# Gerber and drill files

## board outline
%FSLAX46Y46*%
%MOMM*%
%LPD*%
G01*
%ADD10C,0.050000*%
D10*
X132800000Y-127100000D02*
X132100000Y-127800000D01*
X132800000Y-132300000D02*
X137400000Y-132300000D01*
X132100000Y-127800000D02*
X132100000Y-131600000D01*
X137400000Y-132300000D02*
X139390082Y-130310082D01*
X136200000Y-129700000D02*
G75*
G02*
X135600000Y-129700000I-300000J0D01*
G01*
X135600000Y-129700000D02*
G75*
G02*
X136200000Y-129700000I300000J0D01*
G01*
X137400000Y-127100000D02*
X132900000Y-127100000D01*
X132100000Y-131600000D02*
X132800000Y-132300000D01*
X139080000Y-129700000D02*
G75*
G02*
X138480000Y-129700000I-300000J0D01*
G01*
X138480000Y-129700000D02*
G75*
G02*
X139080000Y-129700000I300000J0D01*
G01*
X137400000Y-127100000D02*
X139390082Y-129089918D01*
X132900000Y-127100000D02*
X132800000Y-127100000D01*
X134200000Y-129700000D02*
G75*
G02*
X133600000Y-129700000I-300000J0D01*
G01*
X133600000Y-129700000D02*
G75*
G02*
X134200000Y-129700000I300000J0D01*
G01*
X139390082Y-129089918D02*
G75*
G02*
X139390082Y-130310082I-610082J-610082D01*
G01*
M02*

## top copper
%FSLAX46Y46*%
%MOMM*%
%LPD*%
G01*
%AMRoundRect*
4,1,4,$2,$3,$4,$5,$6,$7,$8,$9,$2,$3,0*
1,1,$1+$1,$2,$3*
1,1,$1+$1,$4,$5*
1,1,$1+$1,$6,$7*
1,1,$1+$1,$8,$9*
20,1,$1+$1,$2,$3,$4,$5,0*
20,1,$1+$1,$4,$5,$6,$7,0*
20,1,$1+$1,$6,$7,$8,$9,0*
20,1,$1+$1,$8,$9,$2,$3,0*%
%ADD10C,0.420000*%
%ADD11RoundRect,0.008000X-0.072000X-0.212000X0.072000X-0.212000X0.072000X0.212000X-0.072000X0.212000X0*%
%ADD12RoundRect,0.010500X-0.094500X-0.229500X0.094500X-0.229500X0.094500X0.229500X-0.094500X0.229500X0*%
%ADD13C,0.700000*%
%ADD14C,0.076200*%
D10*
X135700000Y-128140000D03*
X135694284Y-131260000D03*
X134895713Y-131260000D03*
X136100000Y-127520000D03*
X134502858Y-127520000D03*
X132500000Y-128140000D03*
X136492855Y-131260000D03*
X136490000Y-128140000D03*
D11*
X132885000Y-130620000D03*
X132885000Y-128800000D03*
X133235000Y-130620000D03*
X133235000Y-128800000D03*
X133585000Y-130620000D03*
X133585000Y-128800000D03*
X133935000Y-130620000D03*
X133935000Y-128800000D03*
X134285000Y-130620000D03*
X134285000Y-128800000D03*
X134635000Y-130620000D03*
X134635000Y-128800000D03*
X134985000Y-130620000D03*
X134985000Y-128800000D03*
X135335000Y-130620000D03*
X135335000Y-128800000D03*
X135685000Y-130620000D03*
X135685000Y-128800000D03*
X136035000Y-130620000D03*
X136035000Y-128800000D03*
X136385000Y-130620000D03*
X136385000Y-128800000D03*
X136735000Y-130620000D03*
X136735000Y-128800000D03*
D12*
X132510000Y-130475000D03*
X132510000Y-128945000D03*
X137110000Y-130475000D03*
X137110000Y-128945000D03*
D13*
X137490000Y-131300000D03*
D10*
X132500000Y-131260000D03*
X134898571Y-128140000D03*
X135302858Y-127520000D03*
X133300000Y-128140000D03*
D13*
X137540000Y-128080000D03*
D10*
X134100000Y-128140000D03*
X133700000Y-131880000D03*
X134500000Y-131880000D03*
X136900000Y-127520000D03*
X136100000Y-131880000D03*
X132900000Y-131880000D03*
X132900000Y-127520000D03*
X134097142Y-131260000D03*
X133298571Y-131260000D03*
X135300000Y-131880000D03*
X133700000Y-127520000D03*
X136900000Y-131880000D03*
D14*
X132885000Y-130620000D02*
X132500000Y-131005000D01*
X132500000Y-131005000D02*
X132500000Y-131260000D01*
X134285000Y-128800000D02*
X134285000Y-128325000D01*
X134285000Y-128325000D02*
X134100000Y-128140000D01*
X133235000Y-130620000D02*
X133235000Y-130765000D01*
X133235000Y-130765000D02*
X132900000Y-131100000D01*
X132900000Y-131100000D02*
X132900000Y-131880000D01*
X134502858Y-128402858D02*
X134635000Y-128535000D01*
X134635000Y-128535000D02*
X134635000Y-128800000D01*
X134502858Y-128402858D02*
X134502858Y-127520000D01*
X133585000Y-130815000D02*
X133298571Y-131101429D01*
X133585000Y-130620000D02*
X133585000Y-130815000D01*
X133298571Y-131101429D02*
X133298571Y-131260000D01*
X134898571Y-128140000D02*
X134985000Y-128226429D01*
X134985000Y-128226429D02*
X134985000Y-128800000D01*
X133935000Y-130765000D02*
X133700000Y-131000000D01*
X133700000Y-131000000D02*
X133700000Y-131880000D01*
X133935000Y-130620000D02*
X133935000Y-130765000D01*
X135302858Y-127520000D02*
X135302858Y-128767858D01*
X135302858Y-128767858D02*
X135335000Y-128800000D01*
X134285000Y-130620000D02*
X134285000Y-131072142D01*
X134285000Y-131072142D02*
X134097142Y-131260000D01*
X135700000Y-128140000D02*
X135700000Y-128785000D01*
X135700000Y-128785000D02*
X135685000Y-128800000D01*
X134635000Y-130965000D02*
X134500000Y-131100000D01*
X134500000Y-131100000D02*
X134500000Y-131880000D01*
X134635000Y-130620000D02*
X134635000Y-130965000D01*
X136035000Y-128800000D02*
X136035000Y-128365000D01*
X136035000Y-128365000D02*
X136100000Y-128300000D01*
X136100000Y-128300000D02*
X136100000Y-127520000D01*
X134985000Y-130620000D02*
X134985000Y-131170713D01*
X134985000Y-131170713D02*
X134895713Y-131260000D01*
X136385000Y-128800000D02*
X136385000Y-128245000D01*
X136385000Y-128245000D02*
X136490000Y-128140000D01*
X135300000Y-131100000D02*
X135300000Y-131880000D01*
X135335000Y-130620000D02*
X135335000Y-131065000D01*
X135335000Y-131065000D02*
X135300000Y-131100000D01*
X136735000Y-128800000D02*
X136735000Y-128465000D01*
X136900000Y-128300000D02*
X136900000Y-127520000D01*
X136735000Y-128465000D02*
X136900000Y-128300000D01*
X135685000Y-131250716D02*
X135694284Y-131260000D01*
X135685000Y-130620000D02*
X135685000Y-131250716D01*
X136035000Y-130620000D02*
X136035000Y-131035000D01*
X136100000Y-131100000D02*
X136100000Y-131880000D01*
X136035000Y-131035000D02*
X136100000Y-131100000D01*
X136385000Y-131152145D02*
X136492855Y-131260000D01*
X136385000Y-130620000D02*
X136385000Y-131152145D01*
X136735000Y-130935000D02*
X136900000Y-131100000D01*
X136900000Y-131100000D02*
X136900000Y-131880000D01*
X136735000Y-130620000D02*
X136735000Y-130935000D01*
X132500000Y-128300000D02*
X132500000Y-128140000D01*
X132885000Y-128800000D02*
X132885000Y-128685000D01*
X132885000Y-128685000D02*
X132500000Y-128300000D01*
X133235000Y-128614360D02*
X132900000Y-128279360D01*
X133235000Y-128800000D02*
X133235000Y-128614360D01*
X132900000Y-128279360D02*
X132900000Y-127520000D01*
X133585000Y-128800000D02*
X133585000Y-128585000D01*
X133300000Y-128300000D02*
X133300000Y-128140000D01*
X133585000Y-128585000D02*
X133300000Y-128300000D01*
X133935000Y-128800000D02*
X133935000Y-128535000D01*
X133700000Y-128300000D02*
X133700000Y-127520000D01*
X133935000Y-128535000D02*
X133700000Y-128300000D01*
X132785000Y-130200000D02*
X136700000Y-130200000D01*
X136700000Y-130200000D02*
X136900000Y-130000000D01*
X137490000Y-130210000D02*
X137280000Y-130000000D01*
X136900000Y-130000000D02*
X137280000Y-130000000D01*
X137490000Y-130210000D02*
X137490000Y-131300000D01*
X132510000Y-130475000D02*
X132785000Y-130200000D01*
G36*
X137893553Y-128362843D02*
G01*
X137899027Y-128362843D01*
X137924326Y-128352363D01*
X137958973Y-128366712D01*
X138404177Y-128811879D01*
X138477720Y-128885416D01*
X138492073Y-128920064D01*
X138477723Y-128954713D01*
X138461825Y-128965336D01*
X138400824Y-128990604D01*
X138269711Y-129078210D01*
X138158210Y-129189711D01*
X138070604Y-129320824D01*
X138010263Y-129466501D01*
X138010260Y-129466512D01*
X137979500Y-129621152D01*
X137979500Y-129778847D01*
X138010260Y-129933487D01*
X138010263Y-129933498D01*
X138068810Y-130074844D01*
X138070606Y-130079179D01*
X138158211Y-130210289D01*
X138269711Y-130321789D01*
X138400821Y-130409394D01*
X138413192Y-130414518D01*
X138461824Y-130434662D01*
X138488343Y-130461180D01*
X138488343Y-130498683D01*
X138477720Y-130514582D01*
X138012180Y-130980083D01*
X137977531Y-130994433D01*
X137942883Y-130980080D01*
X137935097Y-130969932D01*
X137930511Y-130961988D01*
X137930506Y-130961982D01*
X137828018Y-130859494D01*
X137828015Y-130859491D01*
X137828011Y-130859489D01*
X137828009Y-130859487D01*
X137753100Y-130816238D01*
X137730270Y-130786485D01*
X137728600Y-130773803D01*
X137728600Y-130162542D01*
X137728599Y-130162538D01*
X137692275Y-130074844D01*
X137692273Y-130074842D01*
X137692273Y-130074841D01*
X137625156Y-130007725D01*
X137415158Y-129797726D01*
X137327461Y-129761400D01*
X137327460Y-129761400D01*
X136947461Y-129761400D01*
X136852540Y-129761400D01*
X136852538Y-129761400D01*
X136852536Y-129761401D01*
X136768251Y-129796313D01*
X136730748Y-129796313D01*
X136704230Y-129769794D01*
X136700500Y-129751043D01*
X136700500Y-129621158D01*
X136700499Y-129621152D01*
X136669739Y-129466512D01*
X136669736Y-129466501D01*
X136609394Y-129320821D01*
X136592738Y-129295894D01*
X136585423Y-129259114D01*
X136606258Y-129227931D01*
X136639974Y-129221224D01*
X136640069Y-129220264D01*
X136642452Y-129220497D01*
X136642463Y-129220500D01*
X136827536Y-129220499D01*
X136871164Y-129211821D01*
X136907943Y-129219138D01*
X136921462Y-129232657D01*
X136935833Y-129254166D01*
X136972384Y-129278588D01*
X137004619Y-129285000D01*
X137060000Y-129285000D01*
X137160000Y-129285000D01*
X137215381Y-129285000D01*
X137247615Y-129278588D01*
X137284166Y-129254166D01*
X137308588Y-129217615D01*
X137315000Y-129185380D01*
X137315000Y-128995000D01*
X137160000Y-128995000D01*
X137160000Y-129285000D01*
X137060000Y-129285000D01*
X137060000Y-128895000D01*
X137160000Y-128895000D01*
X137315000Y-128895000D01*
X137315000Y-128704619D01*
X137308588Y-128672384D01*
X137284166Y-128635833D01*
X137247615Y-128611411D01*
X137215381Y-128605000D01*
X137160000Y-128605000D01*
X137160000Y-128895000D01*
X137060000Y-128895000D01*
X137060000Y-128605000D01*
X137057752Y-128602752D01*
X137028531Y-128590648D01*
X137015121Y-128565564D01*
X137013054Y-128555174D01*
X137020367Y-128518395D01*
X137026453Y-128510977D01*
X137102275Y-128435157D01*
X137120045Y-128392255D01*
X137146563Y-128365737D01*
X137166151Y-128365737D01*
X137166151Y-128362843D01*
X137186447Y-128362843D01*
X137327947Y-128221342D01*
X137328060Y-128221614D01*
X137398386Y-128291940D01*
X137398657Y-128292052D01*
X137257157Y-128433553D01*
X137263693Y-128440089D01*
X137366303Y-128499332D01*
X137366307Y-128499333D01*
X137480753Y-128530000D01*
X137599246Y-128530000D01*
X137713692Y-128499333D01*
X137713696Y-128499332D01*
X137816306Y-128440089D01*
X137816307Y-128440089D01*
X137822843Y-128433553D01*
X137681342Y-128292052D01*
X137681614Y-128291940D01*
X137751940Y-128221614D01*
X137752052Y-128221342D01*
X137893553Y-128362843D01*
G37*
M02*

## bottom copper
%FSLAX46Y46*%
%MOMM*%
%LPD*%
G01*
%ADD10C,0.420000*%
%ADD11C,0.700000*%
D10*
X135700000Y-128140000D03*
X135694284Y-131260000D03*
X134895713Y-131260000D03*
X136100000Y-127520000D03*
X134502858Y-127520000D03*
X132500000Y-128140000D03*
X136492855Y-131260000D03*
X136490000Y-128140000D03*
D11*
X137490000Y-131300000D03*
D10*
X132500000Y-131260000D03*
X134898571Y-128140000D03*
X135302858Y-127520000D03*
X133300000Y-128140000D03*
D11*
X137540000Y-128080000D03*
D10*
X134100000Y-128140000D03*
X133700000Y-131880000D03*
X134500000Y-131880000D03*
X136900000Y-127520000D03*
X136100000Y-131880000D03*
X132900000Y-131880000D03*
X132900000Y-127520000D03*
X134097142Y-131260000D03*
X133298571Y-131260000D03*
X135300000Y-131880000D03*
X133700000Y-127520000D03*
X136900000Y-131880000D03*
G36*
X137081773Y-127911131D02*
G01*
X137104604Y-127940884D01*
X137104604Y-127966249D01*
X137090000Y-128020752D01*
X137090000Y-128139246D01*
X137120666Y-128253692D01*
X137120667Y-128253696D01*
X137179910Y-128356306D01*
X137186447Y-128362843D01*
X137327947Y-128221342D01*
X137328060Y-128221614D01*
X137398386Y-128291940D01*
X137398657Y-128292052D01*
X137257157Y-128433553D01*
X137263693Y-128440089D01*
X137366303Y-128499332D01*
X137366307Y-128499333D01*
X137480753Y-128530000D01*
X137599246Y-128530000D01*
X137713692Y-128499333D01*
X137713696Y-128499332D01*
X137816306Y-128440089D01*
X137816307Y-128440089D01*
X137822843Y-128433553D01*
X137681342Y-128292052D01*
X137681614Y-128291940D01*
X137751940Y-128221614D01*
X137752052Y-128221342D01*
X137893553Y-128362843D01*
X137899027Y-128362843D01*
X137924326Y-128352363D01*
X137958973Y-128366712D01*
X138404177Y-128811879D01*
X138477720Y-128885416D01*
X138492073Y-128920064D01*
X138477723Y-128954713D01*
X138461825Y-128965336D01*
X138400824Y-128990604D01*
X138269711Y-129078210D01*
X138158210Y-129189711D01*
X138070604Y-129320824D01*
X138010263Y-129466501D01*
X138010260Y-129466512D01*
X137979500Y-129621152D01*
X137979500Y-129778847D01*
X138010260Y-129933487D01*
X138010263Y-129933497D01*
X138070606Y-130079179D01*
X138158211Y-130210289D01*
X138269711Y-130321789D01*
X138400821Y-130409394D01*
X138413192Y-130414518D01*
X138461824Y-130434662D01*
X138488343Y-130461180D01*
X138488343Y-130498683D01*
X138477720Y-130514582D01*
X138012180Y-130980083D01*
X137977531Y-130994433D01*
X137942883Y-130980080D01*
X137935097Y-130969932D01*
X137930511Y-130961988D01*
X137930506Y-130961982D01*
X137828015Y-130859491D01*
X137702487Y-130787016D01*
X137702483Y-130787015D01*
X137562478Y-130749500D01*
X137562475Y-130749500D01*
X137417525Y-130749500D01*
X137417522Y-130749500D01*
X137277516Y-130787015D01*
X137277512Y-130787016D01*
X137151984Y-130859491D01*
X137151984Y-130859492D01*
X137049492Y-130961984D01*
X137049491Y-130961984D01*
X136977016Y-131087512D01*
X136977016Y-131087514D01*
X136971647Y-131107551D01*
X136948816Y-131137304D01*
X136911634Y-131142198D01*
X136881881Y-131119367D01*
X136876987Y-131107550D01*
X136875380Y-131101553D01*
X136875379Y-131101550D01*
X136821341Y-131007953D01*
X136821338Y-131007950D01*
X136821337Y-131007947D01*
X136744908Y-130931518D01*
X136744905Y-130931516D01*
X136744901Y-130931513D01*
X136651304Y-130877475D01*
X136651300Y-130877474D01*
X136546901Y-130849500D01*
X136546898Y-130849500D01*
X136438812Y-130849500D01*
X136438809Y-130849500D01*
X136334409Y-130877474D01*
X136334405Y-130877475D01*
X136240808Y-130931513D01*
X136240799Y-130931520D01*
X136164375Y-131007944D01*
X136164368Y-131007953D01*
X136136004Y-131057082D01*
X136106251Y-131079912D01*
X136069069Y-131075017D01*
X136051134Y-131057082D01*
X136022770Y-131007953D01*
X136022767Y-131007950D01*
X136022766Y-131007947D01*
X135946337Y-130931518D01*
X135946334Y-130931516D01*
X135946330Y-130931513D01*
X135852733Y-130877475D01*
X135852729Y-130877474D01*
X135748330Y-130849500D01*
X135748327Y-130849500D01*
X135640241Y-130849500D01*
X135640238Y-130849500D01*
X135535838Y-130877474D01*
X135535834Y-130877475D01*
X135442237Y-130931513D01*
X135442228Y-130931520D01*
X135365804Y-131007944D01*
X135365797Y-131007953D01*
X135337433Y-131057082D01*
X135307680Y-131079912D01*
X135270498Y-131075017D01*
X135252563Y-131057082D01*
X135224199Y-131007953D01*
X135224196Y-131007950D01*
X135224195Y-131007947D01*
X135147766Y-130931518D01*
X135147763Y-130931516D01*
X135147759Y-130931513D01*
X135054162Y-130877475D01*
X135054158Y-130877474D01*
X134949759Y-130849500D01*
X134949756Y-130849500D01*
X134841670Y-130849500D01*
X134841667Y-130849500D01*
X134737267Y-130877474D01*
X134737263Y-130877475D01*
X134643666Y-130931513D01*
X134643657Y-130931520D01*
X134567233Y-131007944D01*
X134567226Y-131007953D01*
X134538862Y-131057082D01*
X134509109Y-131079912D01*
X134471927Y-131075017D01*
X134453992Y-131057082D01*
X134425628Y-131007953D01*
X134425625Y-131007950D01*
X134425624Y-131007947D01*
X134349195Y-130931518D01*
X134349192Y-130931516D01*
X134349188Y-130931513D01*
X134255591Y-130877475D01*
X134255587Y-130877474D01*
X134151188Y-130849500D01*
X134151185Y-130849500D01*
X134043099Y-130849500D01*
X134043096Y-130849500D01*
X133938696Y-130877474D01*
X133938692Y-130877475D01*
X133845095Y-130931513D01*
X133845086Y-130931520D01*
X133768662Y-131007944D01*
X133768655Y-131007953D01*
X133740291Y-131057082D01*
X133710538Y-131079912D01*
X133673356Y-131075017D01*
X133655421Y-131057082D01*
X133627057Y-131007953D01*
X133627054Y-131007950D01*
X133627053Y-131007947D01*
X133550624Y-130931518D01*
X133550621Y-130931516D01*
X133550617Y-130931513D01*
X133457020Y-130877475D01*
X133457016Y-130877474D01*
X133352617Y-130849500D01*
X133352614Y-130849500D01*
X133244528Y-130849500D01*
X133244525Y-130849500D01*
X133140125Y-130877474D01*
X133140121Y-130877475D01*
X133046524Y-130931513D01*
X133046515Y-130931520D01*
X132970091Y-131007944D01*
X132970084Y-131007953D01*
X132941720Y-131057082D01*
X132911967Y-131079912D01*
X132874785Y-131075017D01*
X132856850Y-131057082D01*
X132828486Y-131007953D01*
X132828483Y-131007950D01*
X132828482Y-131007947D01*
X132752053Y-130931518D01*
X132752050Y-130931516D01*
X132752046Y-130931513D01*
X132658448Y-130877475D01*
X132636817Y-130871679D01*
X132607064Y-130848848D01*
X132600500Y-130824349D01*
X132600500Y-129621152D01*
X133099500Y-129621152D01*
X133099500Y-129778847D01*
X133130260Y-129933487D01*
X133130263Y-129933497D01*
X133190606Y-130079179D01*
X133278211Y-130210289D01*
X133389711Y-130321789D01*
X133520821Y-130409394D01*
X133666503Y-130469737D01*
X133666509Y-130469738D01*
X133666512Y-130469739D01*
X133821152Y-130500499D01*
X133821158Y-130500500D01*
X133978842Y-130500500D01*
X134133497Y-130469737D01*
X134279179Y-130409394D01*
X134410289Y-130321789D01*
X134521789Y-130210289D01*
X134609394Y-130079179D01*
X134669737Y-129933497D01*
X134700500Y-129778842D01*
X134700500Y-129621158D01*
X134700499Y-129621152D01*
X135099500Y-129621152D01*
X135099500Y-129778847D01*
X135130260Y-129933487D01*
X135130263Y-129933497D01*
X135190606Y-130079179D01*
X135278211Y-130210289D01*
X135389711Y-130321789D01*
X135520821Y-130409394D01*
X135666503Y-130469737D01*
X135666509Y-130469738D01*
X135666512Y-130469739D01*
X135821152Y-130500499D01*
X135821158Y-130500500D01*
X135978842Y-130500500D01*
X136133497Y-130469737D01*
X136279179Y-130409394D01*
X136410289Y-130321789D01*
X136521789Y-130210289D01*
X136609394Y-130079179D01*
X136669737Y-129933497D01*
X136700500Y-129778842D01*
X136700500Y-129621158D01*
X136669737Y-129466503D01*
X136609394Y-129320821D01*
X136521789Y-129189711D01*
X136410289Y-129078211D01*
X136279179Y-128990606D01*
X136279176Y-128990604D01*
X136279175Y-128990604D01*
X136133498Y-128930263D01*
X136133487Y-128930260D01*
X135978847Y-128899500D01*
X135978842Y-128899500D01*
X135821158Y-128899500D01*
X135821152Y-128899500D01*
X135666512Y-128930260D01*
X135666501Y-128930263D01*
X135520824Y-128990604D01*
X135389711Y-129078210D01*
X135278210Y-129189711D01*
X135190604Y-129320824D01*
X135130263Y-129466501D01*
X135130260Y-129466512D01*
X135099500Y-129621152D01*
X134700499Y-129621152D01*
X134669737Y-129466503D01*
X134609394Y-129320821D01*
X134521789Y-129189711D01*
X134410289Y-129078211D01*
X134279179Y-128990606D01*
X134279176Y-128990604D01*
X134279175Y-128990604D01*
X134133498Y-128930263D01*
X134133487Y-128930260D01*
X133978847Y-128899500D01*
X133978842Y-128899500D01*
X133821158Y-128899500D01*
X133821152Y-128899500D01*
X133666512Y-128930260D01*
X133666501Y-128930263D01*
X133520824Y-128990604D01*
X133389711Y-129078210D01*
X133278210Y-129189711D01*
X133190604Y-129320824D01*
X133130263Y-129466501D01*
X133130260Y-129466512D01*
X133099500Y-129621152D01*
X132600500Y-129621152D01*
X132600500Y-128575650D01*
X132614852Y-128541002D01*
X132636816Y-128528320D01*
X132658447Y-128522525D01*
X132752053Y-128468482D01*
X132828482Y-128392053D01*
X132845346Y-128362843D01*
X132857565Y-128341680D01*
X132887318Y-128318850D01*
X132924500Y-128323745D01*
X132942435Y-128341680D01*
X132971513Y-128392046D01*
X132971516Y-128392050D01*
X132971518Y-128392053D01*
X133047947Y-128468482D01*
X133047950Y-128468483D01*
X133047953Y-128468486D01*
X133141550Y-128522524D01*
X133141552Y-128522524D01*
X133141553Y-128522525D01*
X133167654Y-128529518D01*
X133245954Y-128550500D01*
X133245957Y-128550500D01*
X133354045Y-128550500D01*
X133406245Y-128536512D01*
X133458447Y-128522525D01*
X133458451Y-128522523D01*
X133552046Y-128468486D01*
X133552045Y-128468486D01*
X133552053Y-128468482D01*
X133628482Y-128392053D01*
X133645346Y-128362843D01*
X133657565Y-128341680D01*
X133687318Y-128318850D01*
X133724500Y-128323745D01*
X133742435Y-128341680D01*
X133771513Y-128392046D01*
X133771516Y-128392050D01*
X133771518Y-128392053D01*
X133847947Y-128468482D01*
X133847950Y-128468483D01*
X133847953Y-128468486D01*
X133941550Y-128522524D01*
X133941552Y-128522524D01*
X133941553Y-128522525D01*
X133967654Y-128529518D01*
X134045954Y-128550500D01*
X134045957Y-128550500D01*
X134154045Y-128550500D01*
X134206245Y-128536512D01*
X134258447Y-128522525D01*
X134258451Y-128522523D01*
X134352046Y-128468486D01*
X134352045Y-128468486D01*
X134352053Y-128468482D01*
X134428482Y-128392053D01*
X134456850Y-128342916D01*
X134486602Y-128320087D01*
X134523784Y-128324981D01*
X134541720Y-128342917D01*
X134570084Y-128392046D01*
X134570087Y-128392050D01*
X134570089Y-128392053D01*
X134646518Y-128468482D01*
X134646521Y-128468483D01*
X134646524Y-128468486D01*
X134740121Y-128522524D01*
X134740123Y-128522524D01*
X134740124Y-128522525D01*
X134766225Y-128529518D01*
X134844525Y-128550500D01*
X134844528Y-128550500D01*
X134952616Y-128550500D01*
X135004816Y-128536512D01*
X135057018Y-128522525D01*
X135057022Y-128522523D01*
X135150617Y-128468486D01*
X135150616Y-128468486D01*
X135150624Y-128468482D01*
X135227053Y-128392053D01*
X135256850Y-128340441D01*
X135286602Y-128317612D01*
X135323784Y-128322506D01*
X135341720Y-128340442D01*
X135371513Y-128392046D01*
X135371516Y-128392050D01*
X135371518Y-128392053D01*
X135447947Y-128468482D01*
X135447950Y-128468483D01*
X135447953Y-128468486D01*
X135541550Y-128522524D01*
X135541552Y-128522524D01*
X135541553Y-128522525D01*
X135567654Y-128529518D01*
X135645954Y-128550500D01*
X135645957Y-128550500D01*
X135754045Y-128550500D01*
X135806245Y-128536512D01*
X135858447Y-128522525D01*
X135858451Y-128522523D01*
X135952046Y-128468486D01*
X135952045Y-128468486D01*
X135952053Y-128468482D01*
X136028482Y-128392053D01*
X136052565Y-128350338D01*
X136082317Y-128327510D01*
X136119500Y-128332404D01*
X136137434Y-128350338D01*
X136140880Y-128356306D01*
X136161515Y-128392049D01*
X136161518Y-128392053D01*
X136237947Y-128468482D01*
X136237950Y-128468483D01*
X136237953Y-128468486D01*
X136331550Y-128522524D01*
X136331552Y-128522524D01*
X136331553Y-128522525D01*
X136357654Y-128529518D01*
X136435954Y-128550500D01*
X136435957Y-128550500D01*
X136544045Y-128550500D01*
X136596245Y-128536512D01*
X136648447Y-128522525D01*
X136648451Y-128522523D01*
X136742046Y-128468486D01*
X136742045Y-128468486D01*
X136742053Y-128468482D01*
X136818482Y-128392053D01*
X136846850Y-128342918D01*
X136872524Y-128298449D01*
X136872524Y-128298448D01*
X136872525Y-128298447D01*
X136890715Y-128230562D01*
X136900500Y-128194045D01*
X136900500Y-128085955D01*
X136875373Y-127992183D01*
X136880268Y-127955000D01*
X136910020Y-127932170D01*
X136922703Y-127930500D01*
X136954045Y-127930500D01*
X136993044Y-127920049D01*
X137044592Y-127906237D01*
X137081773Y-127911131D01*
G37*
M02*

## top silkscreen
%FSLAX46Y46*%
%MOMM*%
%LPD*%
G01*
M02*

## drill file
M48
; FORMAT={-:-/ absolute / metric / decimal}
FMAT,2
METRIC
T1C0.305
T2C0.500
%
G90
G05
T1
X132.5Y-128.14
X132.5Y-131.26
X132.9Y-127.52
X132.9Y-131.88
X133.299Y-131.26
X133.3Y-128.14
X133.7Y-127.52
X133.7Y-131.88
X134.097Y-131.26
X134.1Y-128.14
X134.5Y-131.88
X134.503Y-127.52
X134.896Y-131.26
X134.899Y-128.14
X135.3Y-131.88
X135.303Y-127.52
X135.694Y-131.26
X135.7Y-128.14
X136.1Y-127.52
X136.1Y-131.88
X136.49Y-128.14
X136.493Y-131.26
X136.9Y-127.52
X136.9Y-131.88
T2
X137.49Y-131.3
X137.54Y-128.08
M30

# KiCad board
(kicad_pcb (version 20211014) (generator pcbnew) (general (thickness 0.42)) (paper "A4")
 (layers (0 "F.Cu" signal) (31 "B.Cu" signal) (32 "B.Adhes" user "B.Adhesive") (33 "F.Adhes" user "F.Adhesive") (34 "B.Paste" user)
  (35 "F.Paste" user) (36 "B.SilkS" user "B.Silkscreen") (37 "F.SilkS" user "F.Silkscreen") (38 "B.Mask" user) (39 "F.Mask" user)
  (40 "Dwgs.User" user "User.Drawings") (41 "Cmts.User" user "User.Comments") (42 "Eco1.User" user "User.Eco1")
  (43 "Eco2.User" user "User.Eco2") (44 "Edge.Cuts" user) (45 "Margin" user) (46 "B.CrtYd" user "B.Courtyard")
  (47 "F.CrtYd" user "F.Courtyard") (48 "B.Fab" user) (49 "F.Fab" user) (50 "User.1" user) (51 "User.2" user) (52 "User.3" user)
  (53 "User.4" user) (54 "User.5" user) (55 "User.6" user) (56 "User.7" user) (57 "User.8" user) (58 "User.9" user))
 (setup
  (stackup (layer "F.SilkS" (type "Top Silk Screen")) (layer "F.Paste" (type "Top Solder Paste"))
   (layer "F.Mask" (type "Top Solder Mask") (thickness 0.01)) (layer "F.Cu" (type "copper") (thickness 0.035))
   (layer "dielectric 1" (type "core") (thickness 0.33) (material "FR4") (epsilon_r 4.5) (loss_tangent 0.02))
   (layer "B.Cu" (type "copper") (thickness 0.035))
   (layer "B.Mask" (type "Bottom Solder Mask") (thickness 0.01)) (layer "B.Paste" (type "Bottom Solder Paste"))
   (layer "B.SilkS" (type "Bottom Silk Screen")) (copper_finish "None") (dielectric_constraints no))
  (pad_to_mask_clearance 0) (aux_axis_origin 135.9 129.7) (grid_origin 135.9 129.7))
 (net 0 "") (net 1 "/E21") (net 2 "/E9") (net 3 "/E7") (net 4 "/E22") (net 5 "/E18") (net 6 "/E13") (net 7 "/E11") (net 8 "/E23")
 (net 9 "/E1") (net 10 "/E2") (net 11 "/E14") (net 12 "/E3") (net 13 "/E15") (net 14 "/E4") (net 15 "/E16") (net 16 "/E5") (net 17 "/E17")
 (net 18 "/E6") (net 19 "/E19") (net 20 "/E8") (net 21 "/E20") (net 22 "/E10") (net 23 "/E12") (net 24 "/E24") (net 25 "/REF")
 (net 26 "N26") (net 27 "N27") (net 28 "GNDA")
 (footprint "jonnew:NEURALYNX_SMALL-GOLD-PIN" (layer "F.Cu") (at 135.7 128.14)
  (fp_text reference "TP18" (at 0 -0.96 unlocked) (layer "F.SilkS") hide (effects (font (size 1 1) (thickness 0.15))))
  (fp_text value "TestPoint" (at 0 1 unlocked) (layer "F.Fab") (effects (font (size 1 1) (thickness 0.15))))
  (pad "1" thru_hole circle (at 0 0) (size 0.42 0.42) (drill 0.3048) (layers *.Cu *.Mask) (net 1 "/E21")))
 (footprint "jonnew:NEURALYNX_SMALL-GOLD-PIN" (layer "F.Cu") (at 135.694284 131.26)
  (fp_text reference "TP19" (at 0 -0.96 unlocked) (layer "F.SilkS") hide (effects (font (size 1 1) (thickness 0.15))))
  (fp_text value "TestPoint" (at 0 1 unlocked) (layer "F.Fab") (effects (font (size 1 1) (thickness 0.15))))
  (pad "1" thru_hole circle (at 0 0) (size 0.42 0.42) (drill 0.3048) (layers *.Cu *.Mask) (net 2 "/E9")))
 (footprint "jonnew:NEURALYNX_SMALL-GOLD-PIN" (layer "F.Cu") (at 134.895713 131.26)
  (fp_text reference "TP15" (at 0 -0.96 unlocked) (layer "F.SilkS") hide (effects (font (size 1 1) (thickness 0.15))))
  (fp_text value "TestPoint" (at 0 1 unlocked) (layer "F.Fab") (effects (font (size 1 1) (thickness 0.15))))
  (pad "1" thru_hole circle (at 0 0) (size 0.42 0.42) (drill 0.3048) (layers *.Cu *.Mask) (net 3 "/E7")))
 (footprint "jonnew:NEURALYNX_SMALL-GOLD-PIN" (layer "F.Cu") (at 136.1 127.52)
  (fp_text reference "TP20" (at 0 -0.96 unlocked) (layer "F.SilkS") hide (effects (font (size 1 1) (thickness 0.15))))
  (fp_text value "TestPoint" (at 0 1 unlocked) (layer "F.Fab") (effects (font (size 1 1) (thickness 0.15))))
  (pad "1" thru_hole circle (at 0 0) (size 0.42 0.42) (drill 0.3048) (layers *.Cu *.Mask) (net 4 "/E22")))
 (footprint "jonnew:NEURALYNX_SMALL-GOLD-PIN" (layer "F.Cu") (at 134.502858 127.52)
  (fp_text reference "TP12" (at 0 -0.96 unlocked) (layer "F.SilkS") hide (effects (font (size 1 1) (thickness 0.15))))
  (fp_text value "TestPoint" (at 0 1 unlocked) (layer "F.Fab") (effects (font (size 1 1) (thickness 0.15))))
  (pad "1" thru_hole circle (at 0 0) (size 0.42 0.42) (drill 0.3048) (layers *.Cu *.Mask) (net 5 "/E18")))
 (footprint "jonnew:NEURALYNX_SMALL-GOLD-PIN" (layer "F.Cu") (at 132.5 128.14)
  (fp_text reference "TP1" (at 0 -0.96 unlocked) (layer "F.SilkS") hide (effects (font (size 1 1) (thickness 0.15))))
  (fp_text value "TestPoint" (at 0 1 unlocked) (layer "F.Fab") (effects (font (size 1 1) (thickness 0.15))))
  (pad "1" thru_hole circle (at 0 0) (size 0.42 0.42) (drill 0.3048) (layers *.Cu *.Mask) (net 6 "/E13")))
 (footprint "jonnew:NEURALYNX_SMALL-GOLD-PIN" (layer "F.Cu") (at 136.492855 131.26)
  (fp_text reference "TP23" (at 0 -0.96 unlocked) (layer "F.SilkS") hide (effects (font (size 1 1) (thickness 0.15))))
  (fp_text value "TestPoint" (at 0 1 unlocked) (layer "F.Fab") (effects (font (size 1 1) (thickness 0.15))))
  (pad "1" thru_hole circle (at 0 0) (size 0.42 0.42) (drill 0.3048) (layers *.Cu *.Mask) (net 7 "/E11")))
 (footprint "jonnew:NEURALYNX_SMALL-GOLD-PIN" (layer "F.Cu") (at 136.49 128.14)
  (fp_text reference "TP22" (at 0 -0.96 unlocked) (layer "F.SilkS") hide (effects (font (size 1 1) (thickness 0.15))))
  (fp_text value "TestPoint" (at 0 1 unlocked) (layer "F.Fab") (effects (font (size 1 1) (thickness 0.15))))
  (pad "1" thru_hole circle (at 0 0) (size 0.42 0.42) (drill 0.3048) (layers *.Cu *.Mask) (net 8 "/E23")))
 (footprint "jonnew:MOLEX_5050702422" (layer "F.Cu") (at 134.81 129.71)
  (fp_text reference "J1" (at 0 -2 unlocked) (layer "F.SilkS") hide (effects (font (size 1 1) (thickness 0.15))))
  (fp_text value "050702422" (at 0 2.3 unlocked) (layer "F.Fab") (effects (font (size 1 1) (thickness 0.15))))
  (pad "1" smd roundrect (at -1.925 0.91) (size 0.16 0.44) (layers "F.Cu" "F.Paste" "F.Mask") (roundrect_rratio 0.05) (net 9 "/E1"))
  (pad "2" smd roundrect (at -1.925 -0.91) (size 0.16 0.44) (layers "F.Cu" "F.Paste" "F.Mask") (roundrect_rratio 0.05) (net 6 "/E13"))
  (pad "3" smd roundrect (at -1.575 0.91) (size 0.16 0.44) (layers "F.Cu" "F.Paste" "F.Mask") (roundrect_rratio 0.05) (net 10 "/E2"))
  (pad "4" smd roundrect (at -1.575 -0.91) (size 0.16 0.44) (layers "F.Cu" "F.Paste" "F.Mask") (roundrect_rratio 0.05) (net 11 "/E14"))
  (pad "5" smd roundrect (at -1.225 0.91) (size 0.16 0.44) (layers "F.Cu" "F.Paste" "F.Mask") (roundrect_rratio 0.05) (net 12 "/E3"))
  (pad "6" smd roundrect (at -1.225 -0.91) (size 0.16 0.44) (layers "F.Cu" "F.Paste" "F.Mask") (roundrect_rratio 0.05) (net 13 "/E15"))
  (pad "7" smd roundrect (at -0.875 0.91) (size 0.16 0.44) (layers "F.Cu" "F.Paste" "F.Mask") (roundrect_rratio 0.05) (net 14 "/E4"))
  (pad "8" smd roundrect (at -0.875 -0.91) (size 0.16 0.44) (layers "F.Cu" "F.Paste" "F.Mask") (roundrect_rratio 0.05) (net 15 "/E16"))
  (pad "9" smd roundrect (at -0.525 0.91) (size 0.16 0.44) (layers "F.Cu" "F.Paste" "F.Mask") (roundrect_rratio 0.05) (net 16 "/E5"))
  (pad "10" smd roundrect (at -0.525 -0.91) (size 0.16 0.44) (layers "F.Cu" "F.Paste" "F.Mask") (roundrect_rratio 0.05) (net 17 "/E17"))
  (pad "11" smd roundrect (at -0.175 0.91) (size 0.16 0.44) (layers "F.Cu" "F.Paste" "F.Mask") (roundrect_rratio 0.05) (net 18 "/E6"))
  (pad "12" smd roundrect (at -0.175 -0.91) (size 0.16 0.44) (layers "F.Cu" "F.Paste" "F.Mask") (roundrect_rratio 0.05) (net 5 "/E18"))
  (pad "13" smd roundrect (at 0.175 0.91) (size 0.16 0.44) (layers "F.Cu" "F.Paste" "F.Mask") (roundrect_rratio 0.05) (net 3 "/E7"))
  (pad "14" smd roundrect (at 0.175 -0.91) (size 0.16 0.44) (layers "F.Cu" "F.Paste" "F.Mask") (roundrect_rratio 0.05) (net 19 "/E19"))
  (pad "15" smd roundrect (at 0.525 0.91) (size 0.16 0.44) (layers "F.Cu" "F.Paste" "F.Mask") (roundrect_rratio 0.05) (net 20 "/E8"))
  (pad "16" smd roundrect (at 0.525 -0.91) (size 0.16 0.44) (layers "F.Cu" "F.Paste" "F.Mask") (roundrect_rratio 0.05) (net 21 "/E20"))
  (pad "17" smd roundrect (at 0.875 0.91) (size 0.16 0.44) (layers "F.Cu" "F.Paste" "F.Mask") (roundrect_rratio 0.05) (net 2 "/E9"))
  (pad "18" smd roundrect (at 0.875 -0.91) (size 0.16 0.44) (layers "F.Cu" "F.Paste" "F.Mask") (roundrect_rratio 0.05) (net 1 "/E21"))
  (pad "19" smd roundrect (at 1.225 0.91) (size 0.16 0.44) (layers "F.Cu" "F.Paste" "F.Mask") (roundrect_rratio 0.05) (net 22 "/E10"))
  (pad "20" smd roundrect (at 1.225 -0.91) (size 0.16 0.44) (layers "F.Cu" "F.Paste" "F.Mask") (roundrect_rratio 0.05) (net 4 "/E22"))
  (pad "21" smd roundrect (at 1.575 0.91) (size 0.16 0.44) (layers "F.Cu" "F.Paste" "F.Mask") (roundrect_rratio 0.05) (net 7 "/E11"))
  (pad "22" smd roundrect (at 1.575 -0.91) (size 0.16 0.44) (layers "F.Cu" "F.Paste" "F.Mask") (roundrect_rratio 0.05) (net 8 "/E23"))
  (pad "23" smd roundrect (at 1.925 0.91) (size 0.16 0.44) (layers "F.Cu" "F.Paste" "F.Mask") (roundrect_rratio 0.05) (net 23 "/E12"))
  (pad "24" smd roundrect (at 1.925 -0.91) (size 0.16 0.44) (layers "F.Cu" "F.Paste" "F.Mask") (roundrect_rratio 0.05) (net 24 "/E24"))
  (pad "MP1" smd roundrect (at -2.3 0.765) (size 0.21 0.48) (layers "F.Cu" "F.Paste" "F.Mask") (roundrect_rratio 0.05) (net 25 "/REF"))
  (pad "MP2" smd roundrect (at -2.3 -0.765) (size 0.21 0.48) (layers "F.Cu" "F.Paste" "F.Mask") (roundrect_rratio 0.05) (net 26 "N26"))
  (pad "MP3" smd roundrect (at 2.3 0.765) (size 0.21 0.48) (layers "F.Cu" "F.Paste" "F.Mask") (roundrect_rratio 0.05) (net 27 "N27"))
  (pad "MP4" smd roundrect (at 2.3 -0.765) (size 0.21 0.48) (layers "F.Cu" "F.Paste" "F.Mask") (roundrect_rratio 0.05) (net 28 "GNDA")))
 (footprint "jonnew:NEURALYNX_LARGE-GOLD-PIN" (layer "F.Cu") (at 137.49 131.3)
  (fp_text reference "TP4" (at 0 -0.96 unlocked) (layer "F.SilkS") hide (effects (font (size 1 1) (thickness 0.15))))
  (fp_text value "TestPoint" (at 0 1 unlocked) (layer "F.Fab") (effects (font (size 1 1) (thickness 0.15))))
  (pad "1" thru_hole circle (at 0 0) (size 0.7 0.7) (drill 0.5) (layers *.Cu *.Mask) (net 25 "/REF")))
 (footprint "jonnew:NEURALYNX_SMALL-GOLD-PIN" (layer "F.Cu") (at 132.5 131.26)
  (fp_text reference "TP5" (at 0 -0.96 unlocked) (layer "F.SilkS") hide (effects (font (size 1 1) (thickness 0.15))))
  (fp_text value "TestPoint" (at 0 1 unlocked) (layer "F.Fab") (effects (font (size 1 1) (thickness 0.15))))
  (pad "1" thru_hole circle (at 0 0) (size 0.42 0.42) (drill 0.3048) (layers *.Cu *.Mask) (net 9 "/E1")))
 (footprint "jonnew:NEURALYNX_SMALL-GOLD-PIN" (layer "F.Cu") (at 134.898571 128.14)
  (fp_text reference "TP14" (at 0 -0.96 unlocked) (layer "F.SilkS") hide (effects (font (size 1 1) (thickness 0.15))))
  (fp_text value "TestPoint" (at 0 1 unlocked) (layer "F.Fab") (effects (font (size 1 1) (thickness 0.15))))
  (pad "1" thru_hole circle (at 0 0) (size 0.42 0.42) (drill 0.3048) (layers *.Cu *.Mask) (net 19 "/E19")))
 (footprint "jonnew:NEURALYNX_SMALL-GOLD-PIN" (layer "F.Cu") (at 135.302858 127.52)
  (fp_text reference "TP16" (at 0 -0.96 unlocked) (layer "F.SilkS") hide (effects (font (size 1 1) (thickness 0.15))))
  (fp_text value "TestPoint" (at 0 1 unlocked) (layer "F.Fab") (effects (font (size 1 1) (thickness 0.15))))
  (pad "1" thru_hole circle (at 0 0) (size 0.42 0.42) (drill 0.3048) (layers *.Cu *.Mask) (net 21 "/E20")))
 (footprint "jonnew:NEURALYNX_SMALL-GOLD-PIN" (layer "F.Cu") (at 133.3 128.14)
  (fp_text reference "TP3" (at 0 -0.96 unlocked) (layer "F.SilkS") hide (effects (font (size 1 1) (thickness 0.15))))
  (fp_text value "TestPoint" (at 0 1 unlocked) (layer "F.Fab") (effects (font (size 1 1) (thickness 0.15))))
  (pad "1" thru_hole circle (at 0 0) (size 0.42 0.42) (drill 0.3048) (layers *.Cu *.Mask) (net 13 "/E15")))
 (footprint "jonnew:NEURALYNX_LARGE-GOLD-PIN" (layer "F.Cu") (at 137.54 128.08)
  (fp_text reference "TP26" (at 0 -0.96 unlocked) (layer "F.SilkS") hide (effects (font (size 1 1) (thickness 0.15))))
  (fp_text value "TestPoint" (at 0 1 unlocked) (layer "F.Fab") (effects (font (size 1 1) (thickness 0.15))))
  (pad "1" thru_hole circle (at 0 0) (size 0.7 0.7) (drill 0.5) (layers *.Cu *.Mask) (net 28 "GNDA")))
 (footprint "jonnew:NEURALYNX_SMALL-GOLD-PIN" (layer "F.Cu") (at 134.1 128.14)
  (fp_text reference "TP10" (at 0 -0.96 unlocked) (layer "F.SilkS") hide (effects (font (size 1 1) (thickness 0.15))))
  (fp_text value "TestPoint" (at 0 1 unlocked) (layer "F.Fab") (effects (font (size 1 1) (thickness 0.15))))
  (pad "1" thru_hole circle (at 0 0) (size 0.42 0.42) (drill 0.3048) (layers *.Cu *.Mask) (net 17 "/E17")))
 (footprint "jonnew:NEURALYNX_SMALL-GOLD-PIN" (layer "F.Cu") (at 133.7 131.88)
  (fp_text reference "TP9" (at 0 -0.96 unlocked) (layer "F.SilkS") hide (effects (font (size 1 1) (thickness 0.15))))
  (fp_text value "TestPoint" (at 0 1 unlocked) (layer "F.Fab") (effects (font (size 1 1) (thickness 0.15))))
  (pad "1" thru_hole circle (at 0 0) (size 0.42 0.42) (drill 0.3048) (layers *.Cu *.Mask) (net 14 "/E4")))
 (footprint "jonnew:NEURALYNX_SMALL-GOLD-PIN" (layer "F.Cu") (at 134.5 131.88)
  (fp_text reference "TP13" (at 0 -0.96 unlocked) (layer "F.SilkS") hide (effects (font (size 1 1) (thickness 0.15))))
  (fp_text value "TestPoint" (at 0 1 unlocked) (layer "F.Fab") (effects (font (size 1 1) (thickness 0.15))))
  (pad "1" thru_hole circle (at 0 0) (size 0.42 0.42) (drill 0.3048) (layers *.Cu *.Mask) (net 18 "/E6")))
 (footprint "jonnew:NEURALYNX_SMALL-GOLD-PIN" (layer "F.Cu") (at 136.9 127.52)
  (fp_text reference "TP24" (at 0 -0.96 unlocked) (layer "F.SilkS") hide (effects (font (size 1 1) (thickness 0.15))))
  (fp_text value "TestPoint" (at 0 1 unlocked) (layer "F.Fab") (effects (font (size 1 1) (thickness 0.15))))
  (pad "1" thru_hole circle (at 0 0) (size 0.42 0.42) (drill 0.3048) (layers *.Cu *.Mask) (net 24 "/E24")))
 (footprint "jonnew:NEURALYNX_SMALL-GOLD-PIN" (layer "F.Cu") (at 136.1 131.88)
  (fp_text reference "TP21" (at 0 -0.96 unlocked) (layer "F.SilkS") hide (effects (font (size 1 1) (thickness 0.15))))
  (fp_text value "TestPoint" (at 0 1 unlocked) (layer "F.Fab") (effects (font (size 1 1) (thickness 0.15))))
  (pad "1" thru_hole circle (at 0 0) (size 0.42 0.42) (drill 0.3048) (layers *.Cu *.Mask) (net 22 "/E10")))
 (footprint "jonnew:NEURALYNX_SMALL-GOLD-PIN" (layer "F.Cu") (at 132.9 131.88)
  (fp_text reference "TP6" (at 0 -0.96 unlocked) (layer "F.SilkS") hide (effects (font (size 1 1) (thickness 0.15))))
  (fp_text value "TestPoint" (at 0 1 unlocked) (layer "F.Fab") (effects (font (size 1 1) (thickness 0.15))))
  (pad "1" thru_hole circle (at 0 0) (size 0.42 0.42) (drill 0.3048) (layers *.Cu *.Mask) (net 10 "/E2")))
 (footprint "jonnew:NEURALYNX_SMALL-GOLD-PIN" (layer "F.Cu") (at 132.9 127.52)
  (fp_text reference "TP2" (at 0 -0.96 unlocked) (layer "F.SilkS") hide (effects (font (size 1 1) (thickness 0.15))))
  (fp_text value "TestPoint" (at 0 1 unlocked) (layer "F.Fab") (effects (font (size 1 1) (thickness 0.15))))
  (pad "1" thru_hole circle (at 0 0) (size 0.42 0.42) (drill 0.3048) (layers *.Cu *.Mask) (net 11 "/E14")))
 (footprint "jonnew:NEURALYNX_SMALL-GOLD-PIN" (layer "F.Cu") (at 134.097142 131.26)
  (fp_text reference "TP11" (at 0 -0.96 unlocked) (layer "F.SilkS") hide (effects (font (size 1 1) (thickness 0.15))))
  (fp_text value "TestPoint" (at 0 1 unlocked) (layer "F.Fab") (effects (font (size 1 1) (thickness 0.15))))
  (pad "1" thru_hole circle (at 0 0) (size 0.42 0.42) (drill 0.3048) (layers *.Cu *.Mask) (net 16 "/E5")))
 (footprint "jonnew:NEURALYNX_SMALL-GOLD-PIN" (layer "F.Cu") (at 133.298571 131.26)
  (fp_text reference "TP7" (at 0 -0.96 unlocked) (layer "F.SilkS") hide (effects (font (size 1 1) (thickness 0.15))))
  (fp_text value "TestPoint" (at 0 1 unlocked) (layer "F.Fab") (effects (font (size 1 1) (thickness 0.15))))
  (pad "1" thru_hole circle (at 0 0) (size 0.42 0.42) (drill 0.3048) (layers *.Cu *.Mask) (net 12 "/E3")))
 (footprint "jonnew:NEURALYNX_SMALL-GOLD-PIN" (layer "F.Cu") (at 135.3 131.88)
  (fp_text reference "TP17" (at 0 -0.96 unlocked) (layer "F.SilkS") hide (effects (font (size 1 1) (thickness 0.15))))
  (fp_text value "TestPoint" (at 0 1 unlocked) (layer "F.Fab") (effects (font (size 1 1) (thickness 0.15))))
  (pad "1" thru_hole circle (at 0 0) (size 0.42 0.42) (drill 0.3048) (layers *.Cu *.Mask) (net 20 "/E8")))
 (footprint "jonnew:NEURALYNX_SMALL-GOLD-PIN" (layer "F.Cu") (at 133.7 127.52)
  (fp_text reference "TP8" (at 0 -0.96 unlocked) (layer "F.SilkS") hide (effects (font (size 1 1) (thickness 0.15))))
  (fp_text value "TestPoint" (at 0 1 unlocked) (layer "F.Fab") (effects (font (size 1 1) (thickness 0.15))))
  (pad "1" thru_hole circle (at 0 0) (size 0.42 0.42) (drill 0.3048) (layers *.Cu *.Mask) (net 15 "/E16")))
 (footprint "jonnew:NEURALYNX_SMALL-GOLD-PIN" (layer "F.Cu") (at 136.9 131.88)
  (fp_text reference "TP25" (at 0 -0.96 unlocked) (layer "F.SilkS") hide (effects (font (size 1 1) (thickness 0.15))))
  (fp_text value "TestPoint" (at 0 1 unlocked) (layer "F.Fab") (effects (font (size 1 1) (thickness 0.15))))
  (pad "1" thru_hole circle (at 0 0) (size 0.42 0.42) (drill 0.3048) (layers *.Cu *.Mask) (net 23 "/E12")))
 (gr_line (start 132.8 127.1) (end 132.1 127.8) (layer "Edge.Cuts") (width 0.05))
 (gr_line (start 132.8 132.3) (end 137.4 132.3) (layer "Edge.Cuts") (width 0.05))
 (gr_line (start 132.1 127.8) (end 132.1 131.6) (layer "Edge.Cuts") (width 0.05))
 (gr_line (start 137.4 132.3) (end 139.390082 130.310082) (layer "Edge.Cuts") (width 0.05))
 (gr_circle (center 135.9 129.7) (end 136.2 129.7) (layer "Edge.Cuts") (width 0.05) (fill none))
 (gr_line (start 137.4 127.1) (end 132.9 127.1) (layer "Edge.Cuts") (width 0.05))
 (gr_line (start 132.1 131.6) (end 132.8 132.3) (layer "Edge.Cuts") (width 0.05))
 (gr_circle (center 138.78 129.7) (end 139.08 129.7) (layer "Edge.Cuts") (width 0.05) (fill none))
 (gr_line (start 137.4 127.1) (end 139.390082 129.089918) (layer "Edge.Cuts") (width 0.05))
 (gr_line (start 132.9 127.1) (end 132.8 127.1) (layer "Edge.Cuts") (width 0.05))
 (gr_circle (center 133.9 129.7) (end 134.2 129.7) (layer "Edge.Cuts") (width 0.05) (fill none))
 (gr_arc (start 139.390082 129.089918) (mid 139.642786 129.7) (end 139.390082 130.310082) (layer "Edge.Cuts") (width 0.05))
 (segment (start 132.885 130.62) (end 132.5 131.005) (width 0.0762) (layer "F.Cu") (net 9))
 (segment (start 132.5 131.005) (end 132.5 131.26) (width 0.0762) (layer "F.Cu") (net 9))
 (segment (start 134.285 128.8) (end 134.285 128.325) (width 0.0762) (layer "F.Cu") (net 17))
 (segment (start 134.285 128.325) (end 134.1 128.14) (width 0.0762) (layer "F.Cu") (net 17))
 (segment (start 133.235 130.62) (end 133.235 130.765) (width 0.0762) (layer "F.Cu") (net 10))
 (segment (start 133.235 130.765) (end 132.9 131.1) (width 0.0762) (layer "F.Cu") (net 10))
 (segment (start 132.9 131.1) (end 132.9 131.88) (width 0.0762) (layer "F.Cu") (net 10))
 (segment (start 134.502858 128.402858) (end 134.635 128.535) (width 0.0762) (layer "F.Cu") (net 5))
 (segment (start 134.635 128.535) (end 134.635 128.8) (width 0.0762) (layer "F.Cu") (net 5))
 (segment (start 134.502858 128.402858) (end 134.502858 127.52) (width 0.0762) (layer "F.Cu") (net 5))
 (segment (start 133.585 130.815) (end 133.298571 131.101429) (width 0.0762) (layer "F.Cu") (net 12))
 (segment (start 133.585 130.62) (end 133.585 130.815) (width 0.0762) (layer "F.Cu") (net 12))
 (segment (start 133.298571 131.101429) (end 133.298571 131.26) (width 0.0762) (layer "F.Cu") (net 12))
 (segment (start 134.898571 128.14) (end 134.985 128.226429) (width 0.0762) (layer "F.Cu") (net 19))
 (segment (start 134.985 128.226429) (end 134.985 128.8) (width 0.0762) (layer "F.Cu") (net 19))
 (segment (start 133.935 130.765) (end 133.7 131) (width 0.0762) (layer "F.Cu") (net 14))
 (segment (start 133.7 131) (end 133.7 131.88) (width 0.0762) (layer "F.Cu") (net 14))
 (segment (start 133.935 130.62) (end 133.935 130.765) (width 0.0762) (layer "F.Cu") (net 14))
 (segment (start 135.302858 127.52) (end 135.302858 128.767858) (width 0.0762) (layer "F.Cu") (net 21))
 (segment (start 135.302858 128.767858) (end 135.335 128.8) (width 0.0762) (layer "F.Cu") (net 21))
 (segment (start 134.285 130.62) (end 134.285 131.072142) (width 0.0762) (layer "F.Cu") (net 16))
 (segment (start 134.285 131.072142) (end 134.097142 131.26) (width 0.0762) (layer "F.Cu") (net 16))
 (segment (start 135.7 128.14) (end 135.7 128.785) (width 0.0762) (layer "F.Cu") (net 1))
 (segment (start 135.7 128.785) (end 135.685 128.8) (width 0.0762) (layer "F.Cu") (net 1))
 (segment (start 134.635 130.965) (end 134.5 131.1) (width 0.0762) (layer "F.Cu") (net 18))
 (segment (start 134.5 131.1) (end 134.5 131.88) (width 0.0762) (layer "F.Cu") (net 18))
 (segment (start 134.635 130.62) (end 134.635 130.965) (width 0.0762) (layer "F.Cu") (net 18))
 (segment (start 136.035 128.8) (end 136.035 128.365) (width 0.0762) (layer "F.Cu") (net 4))
 (segment (start 136.035 128.365) (end 136.1 128.3) (width 0.0762) (layer "F.Cu") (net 4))
 (segment (start 136.1 128.3) (end 136.1 127.52) (width 0.0762) (layer "F.Cu") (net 4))
 (segment (start 134.985 130.62) (end 134.985 131.170713) (width 0.0762) (layer "F.Cu") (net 3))
 (segment (start 134.985 131.170713) (end 134.895713 131.26) (width 0.0762) (layer "F.Cu") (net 3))
 (segment (start 136.385 128.8) (end 136.385 128.245) (width 0.0762) (layer "F.Cu") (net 8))
 (segment (start 136.385 128.245) (end 136.49 128.14) (width 0.0762) (layer "F.Cu") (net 8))
 (segment (start 135.3 131.1) (end 135.3 131.88) (width 0.0762) (layer "F.Cu") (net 20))
 (segment (start 135.335 130.62) (end 135.335 131.065) (width 0.0762) (layer "F.Cu") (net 20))
 (segment (start 135.335 131.065) (end 135.3 131.1) (width 0.0762) (layer "F.Cu") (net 20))
 (segment (start 136.735 128.8) (end 136.735 128.465) (width 0.0762) (layer "F.Cu") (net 24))
 (segment (start 136.9 128.3) (end 136.9 127.52) (width 0.0762) (layer "F.Cu") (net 24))
 (segment (start 136.735 128.465) (end 136.9 128.3) (width 0.0762) (layer "F.Cu") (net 24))
 (segment (start 135.685 131.250716) (end 135.694284 131.26) (width 0.0762) (layer "F.Cu") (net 2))
 (segment (start 135.685 130.62) (end 135.685 131.250716) (width 0.0762) (layer "F.Cu") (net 2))
 (segment (start 136.035 130.62) (end 136.035 131.035) (width 0.0762) (layer "F.Cu") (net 22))
 (segment (start 136.1 131.1) (end 136.1 131.88) (width 0.0762) (layer "F.Cu") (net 22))
 (segment (start 136.035 131.035) (end 136.1 131.1) (width 0.0762) (layer "F.Cu") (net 22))
 (segment (start 136.385 131.152145) (end 136.492855 131.26) (width 0.0762) (layer "F.Cu") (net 7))
 (segment (start 136.385 130.62) (end 136.385 131.152145) (width 0.0762) (layer "F.Cu") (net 7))
 (segment (start 136.735 130.935) (end 136.9 131.1) (width 0.0762) (layer "F.Cu") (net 23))
 (segment (start 136.9 131.1) (end 136.9 131.88) (width 0.0762) (layer "F.Cu") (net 23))
 (segment (start 136.735 130.62) (end 136.735 130.935) (width 0.0762) (layer "F.Cu") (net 23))
 (segment (start 132.5 128.3) (end 132.5 128.14) (width 0.0762) (layer "F.Cu") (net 6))
 (segment (start 132.885 128.8) (end 132.885 128.685) (width 0.0762) (layer "F.Cu") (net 6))
 (segment (start 132.885 128.685) (end 132.5 128.3) (width 0.0762) (layer "F.Cu") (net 6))
 (segment (start 133.235 128.61436) (end 132.9 128.27936) (width 0.0762) (layer "F.Cu") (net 11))
 (segment (start 133.235 128.8) (end 133.235 128.61436) (width 0.0762) (layer "F.Cu") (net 11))
 (segment (start 132.9 128.27936) (end 132.9 127.52) (width 0.0762) (layer "F.Cu") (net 11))
 (segment (start 133.585 128.8) (end 133.585 128.585) (width 0.0762) (layer "F.Cu") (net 13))
 (segment (start 133.3 128.3) (end 133.3 128.14) (width 0.0762) (layer "F.Cu") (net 13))
 (segment (start 133.585 128.585) (end 133.3 128.3) (width 0.0762) (layer "F.Cu") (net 13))
 (segment (start 133.935 128.8) (end 133.935 128.535) (width 0.0762) (layer "F.Cu") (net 15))
 (segment (start 133.7 128.3) (end 133.7 127.52) (width 0.0762) (layer "F.Cu") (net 15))
 (segment (start 133.935 128.535) (end 133.7 128.3) (width 0.0762) (layer "F.Cu") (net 15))
 (segment (start 132.785 130.2) (end 136.7 130.2) (width 0.0762) (layer "F.Cu") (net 25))
 (segment (start 136.7 130.2) (end 136.9 130) (width 0.0762) (layer "F.Cu") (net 25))
 (segment (start 137.49 130.21) (end 137.28 130) (width 0.0762) (layer "F.Cu") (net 25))
 (segment (start 136.9 130) (end 137.28 130) (width 0.0762) (layer "F.Cu") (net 25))
 (segment (start 137.49 130.21) (end 137.49 131.3) (width 0.0762) (layer "F.Cu") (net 25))
 (segment (start 132.51 130.475) (end 132.785 130.2) (width 0.0762) (layer "F.Cu") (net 25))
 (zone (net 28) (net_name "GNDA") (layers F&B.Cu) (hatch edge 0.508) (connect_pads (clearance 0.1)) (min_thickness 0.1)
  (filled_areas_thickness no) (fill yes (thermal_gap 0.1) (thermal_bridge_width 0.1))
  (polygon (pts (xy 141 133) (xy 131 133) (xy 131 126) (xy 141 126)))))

